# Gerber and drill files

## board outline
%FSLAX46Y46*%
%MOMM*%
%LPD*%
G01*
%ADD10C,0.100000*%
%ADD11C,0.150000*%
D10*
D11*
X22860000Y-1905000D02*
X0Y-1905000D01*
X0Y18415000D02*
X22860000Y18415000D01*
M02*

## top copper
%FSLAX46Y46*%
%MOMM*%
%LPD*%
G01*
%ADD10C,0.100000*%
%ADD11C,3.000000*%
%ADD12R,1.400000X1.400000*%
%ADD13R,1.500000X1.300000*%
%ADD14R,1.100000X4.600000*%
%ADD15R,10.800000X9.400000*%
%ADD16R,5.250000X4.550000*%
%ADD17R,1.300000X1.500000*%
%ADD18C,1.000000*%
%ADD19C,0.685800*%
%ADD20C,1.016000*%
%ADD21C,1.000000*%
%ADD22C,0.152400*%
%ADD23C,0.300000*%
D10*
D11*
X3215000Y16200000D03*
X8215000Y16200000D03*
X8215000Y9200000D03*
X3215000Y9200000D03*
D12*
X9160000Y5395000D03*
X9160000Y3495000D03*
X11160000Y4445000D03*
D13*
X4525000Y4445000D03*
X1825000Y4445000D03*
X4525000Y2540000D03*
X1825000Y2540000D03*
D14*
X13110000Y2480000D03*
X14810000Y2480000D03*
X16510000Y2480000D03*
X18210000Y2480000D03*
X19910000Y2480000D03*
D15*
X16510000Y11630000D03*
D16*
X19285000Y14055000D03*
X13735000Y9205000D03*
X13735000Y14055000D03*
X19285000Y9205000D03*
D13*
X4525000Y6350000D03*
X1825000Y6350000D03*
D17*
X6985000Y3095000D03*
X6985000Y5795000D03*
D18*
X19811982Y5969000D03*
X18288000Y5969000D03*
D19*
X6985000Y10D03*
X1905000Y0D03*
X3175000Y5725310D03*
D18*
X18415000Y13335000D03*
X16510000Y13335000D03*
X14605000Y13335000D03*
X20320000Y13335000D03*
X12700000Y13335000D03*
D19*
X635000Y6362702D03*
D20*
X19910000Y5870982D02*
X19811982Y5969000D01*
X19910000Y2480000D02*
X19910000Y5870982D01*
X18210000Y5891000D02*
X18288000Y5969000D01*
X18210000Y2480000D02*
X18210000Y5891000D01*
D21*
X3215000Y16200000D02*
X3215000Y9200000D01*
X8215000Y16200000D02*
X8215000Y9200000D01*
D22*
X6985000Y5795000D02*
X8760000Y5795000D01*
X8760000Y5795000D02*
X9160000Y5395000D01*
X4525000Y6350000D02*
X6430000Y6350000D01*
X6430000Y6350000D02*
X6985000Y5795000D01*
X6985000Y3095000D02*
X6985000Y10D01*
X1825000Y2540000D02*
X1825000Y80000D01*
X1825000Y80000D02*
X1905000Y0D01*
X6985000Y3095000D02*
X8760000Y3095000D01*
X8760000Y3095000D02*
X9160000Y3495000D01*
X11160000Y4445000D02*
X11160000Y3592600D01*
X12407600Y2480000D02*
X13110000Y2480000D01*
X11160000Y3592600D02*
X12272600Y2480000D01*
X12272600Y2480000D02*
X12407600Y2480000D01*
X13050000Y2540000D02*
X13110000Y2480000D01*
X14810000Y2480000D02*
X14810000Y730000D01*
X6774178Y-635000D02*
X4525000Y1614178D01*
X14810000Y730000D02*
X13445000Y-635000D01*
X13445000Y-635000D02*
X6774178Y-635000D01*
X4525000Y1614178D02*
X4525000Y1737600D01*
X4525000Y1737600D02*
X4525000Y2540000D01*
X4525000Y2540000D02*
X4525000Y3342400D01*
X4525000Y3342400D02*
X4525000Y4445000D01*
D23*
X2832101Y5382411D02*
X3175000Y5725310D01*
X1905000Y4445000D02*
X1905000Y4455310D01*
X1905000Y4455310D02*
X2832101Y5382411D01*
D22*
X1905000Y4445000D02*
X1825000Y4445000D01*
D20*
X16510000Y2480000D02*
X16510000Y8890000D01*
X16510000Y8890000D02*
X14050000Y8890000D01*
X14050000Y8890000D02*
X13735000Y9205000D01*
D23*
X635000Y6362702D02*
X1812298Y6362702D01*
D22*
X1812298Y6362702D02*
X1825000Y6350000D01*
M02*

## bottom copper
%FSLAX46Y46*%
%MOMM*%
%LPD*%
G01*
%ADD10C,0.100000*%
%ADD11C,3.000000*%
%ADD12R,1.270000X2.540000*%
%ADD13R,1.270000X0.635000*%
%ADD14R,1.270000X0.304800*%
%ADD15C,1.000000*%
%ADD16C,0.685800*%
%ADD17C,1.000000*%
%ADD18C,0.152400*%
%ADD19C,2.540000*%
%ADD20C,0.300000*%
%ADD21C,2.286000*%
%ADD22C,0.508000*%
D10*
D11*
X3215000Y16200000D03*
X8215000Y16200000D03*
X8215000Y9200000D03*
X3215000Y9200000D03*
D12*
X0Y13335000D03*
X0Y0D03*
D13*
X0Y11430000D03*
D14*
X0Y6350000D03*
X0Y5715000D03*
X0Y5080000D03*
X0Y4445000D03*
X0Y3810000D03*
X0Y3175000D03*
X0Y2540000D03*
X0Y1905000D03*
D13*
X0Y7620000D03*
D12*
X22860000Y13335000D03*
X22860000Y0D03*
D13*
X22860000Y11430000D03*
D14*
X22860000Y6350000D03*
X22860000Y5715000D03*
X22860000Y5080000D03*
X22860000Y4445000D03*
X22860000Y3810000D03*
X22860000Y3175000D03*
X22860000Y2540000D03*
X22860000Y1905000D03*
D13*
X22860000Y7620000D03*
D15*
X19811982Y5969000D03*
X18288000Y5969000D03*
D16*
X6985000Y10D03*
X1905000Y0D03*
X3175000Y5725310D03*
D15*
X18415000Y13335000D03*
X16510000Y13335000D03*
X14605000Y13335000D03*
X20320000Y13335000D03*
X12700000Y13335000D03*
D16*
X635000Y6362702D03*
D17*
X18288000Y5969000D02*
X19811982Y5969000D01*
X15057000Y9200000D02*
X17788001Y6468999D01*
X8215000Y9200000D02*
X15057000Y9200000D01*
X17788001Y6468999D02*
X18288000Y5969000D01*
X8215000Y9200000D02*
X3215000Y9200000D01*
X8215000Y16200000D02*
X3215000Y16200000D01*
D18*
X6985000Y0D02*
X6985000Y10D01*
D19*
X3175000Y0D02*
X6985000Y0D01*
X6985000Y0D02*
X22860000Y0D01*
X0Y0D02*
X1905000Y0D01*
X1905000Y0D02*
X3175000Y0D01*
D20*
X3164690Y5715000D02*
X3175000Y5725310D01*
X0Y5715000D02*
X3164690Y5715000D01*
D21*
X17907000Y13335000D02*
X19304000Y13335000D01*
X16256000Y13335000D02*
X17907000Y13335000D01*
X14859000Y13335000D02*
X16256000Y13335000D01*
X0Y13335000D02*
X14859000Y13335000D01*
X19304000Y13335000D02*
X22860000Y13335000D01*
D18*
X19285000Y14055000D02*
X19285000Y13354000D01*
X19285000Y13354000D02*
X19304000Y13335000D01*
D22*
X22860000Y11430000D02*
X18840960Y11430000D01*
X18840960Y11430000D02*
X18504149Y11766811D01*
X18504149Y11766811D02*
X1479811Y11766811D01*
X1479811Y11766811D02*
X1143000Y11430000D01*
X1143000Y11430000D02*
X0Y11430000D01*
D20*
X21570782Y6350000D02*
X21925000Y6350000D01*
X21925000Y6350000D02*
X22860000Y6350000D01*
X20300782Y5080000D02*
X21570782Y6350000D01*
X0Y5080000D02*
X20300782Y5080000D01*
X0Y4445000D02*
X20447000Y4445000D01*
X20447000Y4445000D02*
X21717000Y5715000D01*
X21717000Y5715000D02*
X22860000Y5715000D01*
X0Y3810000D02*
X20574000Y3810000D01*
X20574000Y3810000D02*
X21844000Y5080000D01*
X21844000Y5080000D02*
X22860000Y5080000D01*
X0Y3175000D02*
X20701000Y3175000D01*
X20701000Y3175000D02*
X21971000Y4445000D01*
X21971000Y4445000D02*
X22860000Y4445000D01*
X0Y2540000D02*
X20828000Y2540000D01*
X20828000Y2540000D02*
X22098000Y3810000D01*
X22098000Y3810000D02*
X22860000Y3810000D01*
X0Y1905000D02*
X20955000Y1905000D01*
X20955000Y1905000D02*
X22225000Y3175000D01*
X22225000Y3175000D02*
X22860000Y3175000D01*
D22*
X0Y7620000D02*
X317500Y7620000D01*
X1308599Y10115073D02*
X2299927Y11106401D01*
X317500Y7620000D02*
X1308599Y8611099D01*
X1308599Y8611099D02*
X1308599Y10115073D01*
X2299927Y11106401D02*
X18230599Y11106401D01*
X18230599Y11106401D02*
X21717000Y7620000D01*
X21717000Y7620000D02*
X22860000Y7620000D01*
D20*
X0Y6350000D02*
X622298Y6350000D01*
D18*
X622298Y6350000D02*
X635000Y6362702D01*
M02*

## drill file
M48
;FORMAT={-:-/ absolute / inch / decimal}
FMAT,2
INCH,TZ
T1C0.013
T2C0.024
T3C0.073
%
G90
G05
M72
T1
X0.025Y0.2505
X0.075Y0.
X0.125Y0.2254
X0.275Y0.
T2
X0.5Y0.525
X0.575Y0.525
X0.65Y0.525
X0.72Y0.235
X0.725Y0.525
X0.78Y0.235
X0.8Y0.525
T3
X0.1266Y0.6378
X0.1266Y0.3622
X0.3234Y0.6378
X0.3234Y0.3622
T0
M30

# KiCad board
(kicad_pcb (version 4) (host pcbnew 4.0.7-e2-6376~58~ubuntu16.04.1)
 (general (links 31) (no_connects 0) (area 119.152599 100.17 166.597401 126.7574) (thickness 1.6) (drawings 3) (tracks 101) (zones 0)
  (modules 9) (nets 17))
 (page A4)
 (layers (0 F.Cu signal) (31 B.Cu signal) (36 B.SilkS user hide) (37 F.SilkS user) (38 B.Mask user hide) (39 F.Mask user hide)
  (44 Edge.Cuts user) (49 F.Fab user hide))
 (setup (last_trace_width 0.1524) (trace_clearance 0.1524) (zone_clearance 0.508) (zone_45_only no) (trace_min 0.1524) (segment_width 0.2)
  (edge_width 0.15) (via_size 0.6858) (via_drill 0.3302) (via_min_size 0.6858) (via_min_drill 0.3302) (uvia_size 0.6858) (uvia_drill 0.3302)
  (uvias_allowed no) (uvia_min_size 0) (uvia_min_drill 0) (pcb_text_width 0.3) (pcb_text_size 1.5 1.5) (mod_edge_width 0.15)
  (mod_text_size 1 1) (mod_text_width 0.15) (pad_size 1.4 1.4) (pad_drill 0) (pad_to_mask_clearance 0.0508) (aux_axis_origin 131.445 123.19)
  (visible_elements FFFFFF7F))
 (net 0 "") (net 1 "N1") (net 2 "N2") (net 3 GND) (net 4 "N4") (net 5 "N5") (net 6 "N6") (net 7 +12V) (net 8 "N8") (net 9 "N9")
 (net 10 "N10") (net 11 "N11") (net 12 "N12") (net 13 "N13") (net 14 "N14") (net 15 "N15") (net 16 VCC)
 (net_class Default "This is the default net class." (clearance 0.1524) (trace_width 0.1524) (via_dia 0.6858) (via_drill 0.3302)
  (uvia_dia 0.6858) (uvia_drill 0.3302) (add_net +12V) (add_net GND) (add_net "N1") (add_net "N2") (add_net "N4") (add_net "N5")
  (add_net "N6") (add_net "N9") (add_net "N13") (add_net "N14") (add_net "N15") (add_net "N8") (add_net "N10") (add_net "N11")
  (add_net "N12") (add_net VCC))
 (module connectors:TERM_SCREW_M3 (layer F.Cu) (at 137.16 110.49)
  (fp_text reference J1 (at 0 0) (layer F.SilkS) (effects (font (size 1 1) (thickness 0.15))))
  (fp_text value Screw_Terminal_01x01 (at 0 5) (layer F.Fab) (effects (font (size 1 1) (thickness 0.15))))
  (pad 1 thru_hole circle (at -2.5 -3.5) (size 3 3) (drill 1.85) (layers *.Cu *.Mask) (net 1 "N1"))
  (pad 1 thru_hole circle (at 2.5 -3.5) (size 3 3) (drill 1.85) (layers *.Cu *.Mask) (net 1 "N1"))
  (pad 1 thru_hole circle (at 2.5 3.5) (size 3 3) (drill 1.85) (layers *.Cu *.Mask) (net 1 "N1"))
  (pad 1 thru_hole circle (at -2.5 3.5) (size 3 3) (drill 1.85) (layers *.Cu *.Mask) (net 1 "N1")))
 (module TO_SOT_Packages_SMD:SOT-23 (layer F.Cu) (at 141.605 118.745)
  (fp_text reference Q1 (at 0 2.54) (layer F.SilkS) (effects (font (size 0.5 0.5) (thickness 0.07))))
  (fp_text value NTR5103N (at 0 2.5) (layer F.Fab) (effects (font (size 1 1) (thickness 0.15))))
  (pad 1 smd rect (at -1 -0.95) (size 1.4 1.4) (layers F.Cu F.Mask) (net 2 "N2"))
  (pad 2 smd rect (at -1 0.95) (size 1.4 1.4) (layers F.Cu F.Mask) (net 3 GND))
  (pad 3 smd rect (at 1 0) (size 1.4 1.4) (layers F.Cu F.Mask) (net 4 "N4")))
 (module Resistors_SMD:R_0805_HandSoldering (layer F.Cu) (at 134.62 118.745 180)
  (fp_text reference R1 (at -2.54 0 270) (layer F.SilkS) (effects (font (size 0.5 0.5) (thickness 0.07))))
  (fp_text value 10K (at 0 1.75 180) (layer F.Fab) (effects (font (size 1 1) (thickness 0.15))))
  (pad 1 smd rect (at -1.35 0 180) (size 1.5 1.3) (layers F.Cu F.Mask) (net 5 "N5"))
  (pad 2 smd rect (at 1.35 0 180) (size 1.5 1.3) (layers F.Cu F.Mask) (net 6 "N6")))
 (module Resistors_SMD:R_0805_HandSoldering (layer F.Cu) (at 134.62 120.65 180)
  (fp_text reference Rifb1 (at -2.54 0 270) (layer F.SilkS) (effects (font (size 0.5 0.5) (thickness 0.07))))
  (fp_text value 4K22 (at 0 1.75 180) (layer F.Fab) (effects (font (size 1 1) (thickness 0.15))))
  (pad 1 smd rect (at -1.35 0 180) (size 1.5 1.3) (layers F.Cu F.Mask) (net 5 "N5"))
  (pad 2 smd rect (at 1.35 0 180) (size 1.5 1.3) (layers F.Cu F.Mask) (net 3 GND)))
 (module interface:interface (layer F.Cu) (at 131.445 105.41)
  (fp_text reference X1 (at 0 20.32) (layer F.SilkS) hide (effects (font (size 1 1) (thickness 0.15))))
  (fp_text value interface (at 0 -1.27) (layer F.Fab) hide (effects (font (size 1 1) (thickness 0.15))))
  (pad 1 smd rect (at 0 4.445) (size 1.27 2.54) (layers B.Cu) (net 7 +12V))
  (pad 2 smd rect (at 0 17.78) (size 1.27 2.54) (layers B.Cu) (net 3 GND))
  (pad 3 smd rect (at 0 6.35) (size 1.27 0.635) (layers B.Cu) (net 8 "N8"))
  (pad 5 smd rect (at 0 11.43) (size 1.27 0.3048) (layers B.Cu) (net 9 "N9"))
  (pad 6 smd rect (at 0 12.065) (size 1.27 0.3048) (layers B.Cu) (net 6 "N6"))
  (pad 7 smd rect (at 0 12.7) (size 1.27 0.3048) (layers B.Cu) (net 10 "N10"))
  (pad 8 smd rect (at 0 13.335) (size 1.27 0.3048) (layers B.Cu) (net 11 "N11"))
  (pad 9 smd rect (at 0 13.97) (size 1.27 0.3048) (layers B.Cu) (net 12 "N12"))
  (pad 10 smd rect (at 0 14.605) (size 1.27 0.3048) (layers B.Cu) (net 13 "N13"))
  (pad 11 smd rect (at 0 15.24) (size 1.27 0.3048) (layers B.Cu) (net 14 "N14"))
  (pad 12 smd rect (at 0 15.875) (size 1.27 0.3048) (layers B.Cu) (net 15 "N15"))
  (pad 4 smd rect (at 0 10.16) (size 1.27 0.635) (layers B.Cu) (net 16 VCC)))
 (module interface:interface (layer F.Cu) (at 154.305 105.41)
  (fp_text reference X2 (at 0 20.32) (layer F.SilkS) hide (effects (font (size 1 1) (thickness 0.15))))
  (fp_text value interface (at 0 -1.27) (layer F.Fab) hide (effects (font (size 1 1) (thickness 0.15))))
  (pad 1 smd rect (at 0 4.445) (size 1.27 2.54) (layers B.Cu) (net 7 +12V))
  (pad 2 smd rect (at 0 17.78) (size 1.27 2.54) (layers B.Cu) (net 3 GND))
  (pad 3 smd rect (at 0 6.35) (size 1.27 0.635) (layers B.Cu) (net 8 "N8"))
  (pad 5 smd rect (at 0 11.43) (size 1.27 0.3048) (layers B.Cu) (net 10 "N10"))
  (pad 6 smd rect (at 0 12.065) (size 1.27 0.3048) (layers B.Cu) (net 11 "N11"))
  (pad 7 smd rect (at 0 12.7) (size 1.27 0.3048) (layers B.Cu) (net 12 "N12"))
  (pad 8 smd rect (at 0 13.335) (size 1.27 0.3048) (layers B.Cu) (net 13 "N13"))
  (pad 9 smd rect (at 0 13.97) (size 1.27 0.3048) (layers B.Cu) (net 14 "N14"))
  (pad 10 smd rect (at 0 14.605) (size 1.27 0.3048) (layers B.Cu) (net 15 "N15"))
  (pad 11 smd rect (at 0 15.24) (size 1.27 0.3048) (layers B.Cu))
  (pad 12 smd rect (at 0 15.875) (size 1.27 0.3048) (layers B.Cu))
  (pad 4 smd rect (at 0 10.16) (size 1.27 0.635) (layers B.Cu) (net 16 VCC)))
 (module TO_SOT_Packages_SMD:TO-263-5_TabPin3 (layer F.Cu) (at 147.955 114.935 90)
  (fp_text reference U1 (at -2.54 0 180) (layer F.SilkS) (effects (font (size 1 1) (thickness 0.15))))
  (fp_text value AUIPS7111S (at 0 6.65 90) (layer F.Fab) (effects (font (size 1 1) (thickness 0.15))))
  (pad 1 smd rect (at -5.775 -3.4 90) (size 4.6 1.1) (layers F.Cu F.Mask) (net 4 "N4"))
  (pad 2 smd rect (at -5.775 -1.7 90) (size 4.6 1.1) (layers F.Cu F.Mask) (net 5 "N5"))
  (pad 3 smd rect (at -5.775 0 90) (size 4.6 1.1) (layers F.Cu F.Mask) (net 7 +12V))
  (pad 4 smd rect (at -5.775 1.7 90) (size 4.6 1.1) (layers F.Cu F.Mask) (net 1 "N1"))
  (pad 5 smd rect (at -5.775 3.4 90) (size 4.6 1.1) (layers F.Cu F.Mask) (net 1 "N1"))
  (pad 3 smd rect (at 3.375 0 90) (size 9.4 10.8) (layers F.Cu F.Mask) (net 7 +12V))
  (pad 3 smd rect (at 5.8 2.775 90) (size 4.55 5.25) (layers F.Cu) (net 7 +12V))
  (pad 3 smd rect (at 0.95 -2.775 90) (size 4.55 5.25) (layers F.Cu) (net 7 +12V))
  (pad 3 smd rect (at 5.8 -2.775 90) (size 4.55 5.25) (layers F.Cu) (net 7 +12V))
  (pad 3 smd rect (at 0.95 2.775 90) (size 4.55 5.25) (layers F.Cu) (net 7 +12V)))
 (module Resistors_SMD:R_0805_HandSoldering (layer F.Cu) (at 134.62 116.84 180)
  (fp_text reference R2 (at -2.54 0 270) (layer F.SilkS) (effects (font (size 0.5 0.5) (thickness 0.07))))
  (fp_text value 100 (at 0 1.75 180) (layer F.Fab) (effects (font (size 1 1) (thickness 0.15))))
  (pad 1 smd rect (at -1.35 0 180) (size 1.5 1.3) (layers F.Cu F.Mask) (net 2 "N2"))
  (pad 2 smd rect (at 1.35 0 180) (size 1.5 1.3) (layers F.Cu F.Mask) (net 9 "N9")))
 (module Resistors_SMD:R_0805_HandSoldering (layer F.Cu) (at 138.43 118.745 90)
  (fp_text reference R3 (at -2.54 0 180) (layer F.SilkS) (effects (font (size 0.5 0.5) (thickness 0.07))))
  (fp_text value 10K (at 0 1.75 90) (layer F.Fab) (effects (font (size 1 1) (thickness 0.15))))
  (pad 1 smd rect (at -1.35 0 90) (size 1.5 1.3) (layers F.Cu F.Mask) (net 3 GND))
  (pad 2 smd rect (at 1.35 0 90) (size 1.5 1.3) (layers F.Cu F.Mask) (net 2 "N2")))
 (gr_line (start 154.305 125.095) (end 131.445 125.095) (layer Edge.Cuts) (width 0.15))
 (gr_line (start 131.445 104.775) (end 154.305 104.775) (layer Edge.Cuts) (width 0.15))
 (segment (start 149.733 117.221) (end 151.256982 117.221) (width 1) (layer B.Cu) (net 1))
 (segment (start 151.355 117.319018) (end 151.256982 117.221) (width 1.016) (layer F.Cu) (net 1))
 (segment (start 151.355 120.71) (end 151.355 117.319018) (width 1.016) (layer F.Cu) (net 1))
 (via (at 151.256982 117.221) (size 1) (drill 0.6) (layers F.Cu B.Cu) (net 1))
 (segment (start 149.655 117.299) (end 149.733 117.221) (width 1.016) (layer F.Cu) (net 1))
 (segment (start 146.502 113.99) (end 149.233001 116.721001) (width 1) (layer B.Cu) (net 1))
 (segment (start 139.66 113.99) (end 146.502 113.99) (width 1) (layer B.Cu) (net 1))
 (segment (start 149.655 120.71) (end 149.655 117.299) (width 1.016) (layer F.Cu) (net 1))
 (segment (start 149.233001 116.721001) (end 149.733 117.221) (width 1) (layer B.Cu) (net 1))
 (via (at 149.733 117.221) (size 1) (drill 0.6) (layers F.Cu B.Cu) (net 1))
 (segment (start 134.66 106.99) (end 134.66 113.99) (width 1) (layer F.Cu) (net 1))
 (segment (start 139.66 106.99) (end 139.66 113.99) (width 1) (layer F.Cu) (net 1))
 (segment (start 139.66 113.99) (end 134.66 113.99) (width 1) (layer B.Cu) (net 1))
 (segment (start 139.66 106.99) (end 134.66 106.99) (width 1) (layer B.Cu) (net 1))
 (segment (start 138.43 117.395) (end 140.205 117.395) (width 0.1524) (layer F.Cu) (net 2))
 (segment (start 140.205 117.395) (end 140.605 117.795) (width 0.1524) (layer F.Cu) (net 2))
 (segment (start 135.97 116.84) (end 137.875 116.84) (width 0.1524) (layer F.Cu) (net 2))
 (segment (start 137.875 116.84) (end 138.43 117.395) (width 0.1524) (layer F.Cu) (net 2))
 (segment (start 138.43 120.095) (end 138.43 123.18999) (width 0.1524) (layer F.Cu) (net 3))
 (segment (start 138.43 123.19) (end 138.43 123.18999) (width 0.1524) (layer B.Cu) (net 3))
 (via (at 138.43 123.18999) (size 0.6858) (drill 0.3302) (layers F.Cu B.Cu) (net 3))
 (segment (start 134.62 123.19) (end 138.43 123.19) (width 2.54) (layer B.Cu) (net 3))
 (segment (start 138.43 123.19) (end 154.305 123.19) (width 2.54) (layer B.Cu) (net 3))
 (segment (start 131.445 123.19) (end 133.35 123.19) (width 2.54) (layer B.Cu) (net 3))
 (segment (start 133.35 123.19) (end 134.62 123.19) (width 2.54) (layer B.Cu) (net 3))
 (segment (start 133.27 120.65) (end 133.27 123.11) (width 0.1524) (layer F.Cu) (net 3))
 (via (at 133.35 123.19) (size 0.6858) (drill 0.3302) (layers F.Cu B.Cu) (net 3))
 (segment (start 133.27 123.11) (end 133.35 123.19) (width 0.1524) (layer F.Cu) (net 3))
 (segment (start 138.43 120.095) (end 140.205 120.095) (width 0.1524) (layer F.Cu) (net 3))
 (segment (start 140.205 120.095) (end 140.605 119.695) (width 0.1524) (layer F.Cu) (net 3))
 (segment (start 142.605 118.745) (end 142.605 119.5974) (width 0.1524) (layer F.Cu) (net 4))
 (segment (start 143.8526 120.71) (end 144.555 120.71) (width 0.1524) (layer F.Cu) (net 4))
 (segment (start 142.605 119.5974) (end 143.7176 120.71) (width 0.1524) (layer F.Cu) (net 4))
 (segment (start 143.7176 120.71) (end 143.8526 120.71) (width 0.1524) (layer F.Cu) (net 4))
 (segment (start 144.495 120.65) (end 144.555 120.71) (width 0.1524) (layer F.Cu) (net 4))
 (segment (start 146.255 120.71) (end 146.255 122.46) (width 0.1524) (layer F.Cu) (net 5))
 (segment (start 138.219178 123.825) (end 135.97 121.575822) (width 0.1524) (layer F.Cu) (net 5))
 (segment (start 146.255 122.46) (end 144.89 123.825) (width 0.1524) (layer F.Cu) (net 5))
 (segment (start 144.89 123.825) (end 138.219178 123.825) (width 0.1524) (layer F.Cu) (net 5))
 (segment (start 135.97 121.575822) (end 135.97 121.4524) (width 0.1524) (layer F.Cu) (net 5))
 (segment (start 135.97 121.4524) (end 135.97 120.65) (width 0.1524) (layer F.Cu) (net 5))
 (segment (start 135.97 120.65) (end 135.97 119.8476) (width 0.1524) (layer F.Cu) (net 5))
 (segment (start 135.97 119.8476) (end 135.97 118.745) (width 0.1524) (layer F.Cu) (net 5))
 (segment (start 134.60969 117.475) (end 134.62 117.46469) (width 0.3) (layer B.Cu) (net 6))
 (segment (start 131.445 117.475) (end 134.60969 117.475) (width 0.3) (layer B.Cu) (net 6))
 (segment (start 134.277101 117.807589) (end 134.62 117.46469) (width 0.3) (layer F.Cu) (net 6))
 (segment (start 133.35 118.745) (end 133.35 118.73469) (width 0.3) (layer F.Cu) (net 6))
 (segment (start 133.35 118.73469) (end 134.277101 117.807589) (width 0.3) (layer F.Cu) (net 6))
 (via (at 134.62 117.46469) (size 0.6858) (drill 0.3302) (layers F.Cu B.Cu) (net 6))
 (segment (start 133.35 118.745) (end 133.27 118.745) (width 0.1524) (layer F.Cu) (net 6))
 (segment (start 149.352 109.855) (end 150.749 109.855) (width 2.286) (layer B.Cu) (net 7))
 (via (at 149.86 109.855) (size 1) (drill 0.6) (layers F.Cu B.Cu) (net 7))
 (segment (start 147.701 109.855) (end 149.352 109.855) (width 2.286) (layer B.Cu) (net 7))
 (segment (start 146.304 109.855) (end 147.701 109.855) (width 2.286) (layer B.Cu) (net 7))
 (via (at 147.955 109.855) (size 1) (drill 0.6) (layers F.Cu B.Cu) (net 7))
 (segment (start 131.445 109.855) (end 146.304 109.855) (width 2.286) (layer B.Cu) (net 7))
 (via (at 146.05 109.855) (size 1) (drill 0.6) (layers F.Cu B.Cu) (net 7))
 (segment (start 150.749 109.855) (end 154.305 109.855) (width 2.286) (layer B.Cu) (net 7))
 (segment (start 150.73 109.135) (end 150.73 109.836) (width 0.1524) (layer B.Cu) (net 7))
 (segment (start 150.73 109.836) (end 150.749 109.855) (width 0.1524) (layer B.Cu) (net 7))
 (via (at 151.765 109.855) (size 1) (drill 0.6) (layers F.Cu B.Cu) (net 7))
 (via (at 144.145 109.855) (size 1) (drill 0.6) (layers F.Cu B.Cu) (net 7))
 (segment (start 147.955 120.71) (end 147.955 114.3) (width 1.016) (layer F.Cu) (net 7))
 (segment (start 147.955 114.3) (end 145.495 114.3) (width 1.016) (layer F.Cu) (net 7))
 (segment (start 145.495 114.3) (end 145.18 113.985) (width 1.016) (layer F.Cu) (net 7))
 (segment (start 154.305 111.76) (end 150.28596 111.76) (width 0.508) (layer B.Cu) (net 8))
 (segment (start 150.28596 111.76) (end 149.949149 111.423189) (width 0.508) (layer B.Cu) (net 8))
 (segment (start 149.949149 111.423189) (end 132.924811 111.423189) (width 0.508) (layer B.Cu) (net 8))
 (segment (start 132.924811 111.423189) (end 132.588 111.76) (width 0.508) (layer B.Cu) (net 8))
 (segment (start 132.588 111.76) (end 131.445 111.76) (width 0.508) (layer B.Cu) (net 8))
 (segment (start 153.015782 116.84) (end 153.37 116.84) (width 0.3) (layer B.Cu) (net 10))
 (segment (start 153.37 116.84) (end 154.305 116.84) (width 0.3) (layer B.Cu) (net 10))
 (segment (start 151.745782 118.11) (end 153.015782 116.84) (width 0.3) (layer B.Cu) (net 10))
 (segment (start 131.445 118.11) (end 151.745782 118.11) (width 0.3) (layer B.Cu) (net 10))
 (segment (start 131.445 118.745) (end 151.892 118.745) (width 0.3) (layer B.Cu) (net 11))
 (segment (start 151.892 118.745) (end 153.162 117.475) (width 0.3) (layer B.Cu) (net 11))
 (segment (start 153.162 117.475) (end 154.305 117.475) (width 0.3) (layer B.Cu) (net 11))
 (segment (start 131.445 119.38) (end 152.019 119.38) (width 0.3) (layer B.Cu) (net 12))
 (segment (start 152.019 119.38) (end 153.289 118.11) (width 0.3) (layer B.Cu) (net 12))
 (segment (start 153.289 118.11) (end 154.305 118.11) (width 0.3) (layer B.Cu) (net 12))
 (segment (start 131.445 120.015) (end 152.146 120.015) (width 0.3) (layer B.Cu) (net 13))
 (segment (start 152.146 120.015) (end 153.416 118.745) (width 0.3) (layer B.Cu) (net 13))
 (segment (start 153.416 118.745) (end 154.305 118.745) (width 0.3) (layer B.Cu) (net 13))
 (segment (start 131.445 120.65) (end 152.273 120.65) (width 0.3) (layer B.Cu) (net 14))
 (segment (start 152.273 120.65) (end 153.543 119.38) (width 0.3) (layer B.Cu) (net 14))
 (segment (start 153.543 119.38) (end 154.305 119.38) (width 0.3) (layer B.Cu) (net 14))
 (segment (start 131.445 121.285) (end 152.4 121.285) (width 0.3) (layer B.Cu) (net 15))
 (segment (start 152.4 121.285) (end 153.67 120.015) (width 0.3) (layer B.Cu) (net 15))
 (segment (start 153.67 120.015) (end 154.305 120.015) (width 0.3) (layer B.Cu) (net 15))
 (segment (start 131.445 115.57) (end 131.7625 115.57) (width 0.508) (layer B.Cu) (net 16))
 (segment (start 132.753599 113.074927) (end 133.744927 112.083599) (width 0.508) (layer B.Cu) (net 16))
 (segment (start 131.7625 115.57) (end 132.753599 114.578901) (width 0.508) (layer B.Cu) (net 16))
 (segment (start 132.753599 114.578901) (end 132.753599 113.074927) (width 0.508) (layer B.Cu) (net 16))
 (segment (start 133.744927 112.083599) (end 149.675599 112.083599) (width 0.508) (layer B.Cu) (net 16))
 (segment (start 149.675599 112.083599) (end 153.162 115.57) (width 0.508) (layer B.Cu) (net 16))
 (segment (start 153.162 115.57) (end 154.305 115.57) (width 0.508) (layer B.Cu) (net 16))
 (segment (start 132.08 116.827298) (end 133.257298 116.827298) (width 0.3) (layer F.Cu) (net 9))
 (segment (start 133.257298 116.827298) (end 133.27 116.84) (width 0.1524) (layer F.Cu) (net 9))
 (segment (start 131.445 116.84) (end 132.067298 116.84) (width 0.3) (layer B.Cu) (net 9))
 (segment (start 132.067298 116.84) (end 132.08 116.827298) (width 0.1524) (layer B.Cu) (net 9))
 (via (at 132.08 116.827298) (size 0.6858) (drill 0.3302) (layers F.Cu B.Cu) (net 9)))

